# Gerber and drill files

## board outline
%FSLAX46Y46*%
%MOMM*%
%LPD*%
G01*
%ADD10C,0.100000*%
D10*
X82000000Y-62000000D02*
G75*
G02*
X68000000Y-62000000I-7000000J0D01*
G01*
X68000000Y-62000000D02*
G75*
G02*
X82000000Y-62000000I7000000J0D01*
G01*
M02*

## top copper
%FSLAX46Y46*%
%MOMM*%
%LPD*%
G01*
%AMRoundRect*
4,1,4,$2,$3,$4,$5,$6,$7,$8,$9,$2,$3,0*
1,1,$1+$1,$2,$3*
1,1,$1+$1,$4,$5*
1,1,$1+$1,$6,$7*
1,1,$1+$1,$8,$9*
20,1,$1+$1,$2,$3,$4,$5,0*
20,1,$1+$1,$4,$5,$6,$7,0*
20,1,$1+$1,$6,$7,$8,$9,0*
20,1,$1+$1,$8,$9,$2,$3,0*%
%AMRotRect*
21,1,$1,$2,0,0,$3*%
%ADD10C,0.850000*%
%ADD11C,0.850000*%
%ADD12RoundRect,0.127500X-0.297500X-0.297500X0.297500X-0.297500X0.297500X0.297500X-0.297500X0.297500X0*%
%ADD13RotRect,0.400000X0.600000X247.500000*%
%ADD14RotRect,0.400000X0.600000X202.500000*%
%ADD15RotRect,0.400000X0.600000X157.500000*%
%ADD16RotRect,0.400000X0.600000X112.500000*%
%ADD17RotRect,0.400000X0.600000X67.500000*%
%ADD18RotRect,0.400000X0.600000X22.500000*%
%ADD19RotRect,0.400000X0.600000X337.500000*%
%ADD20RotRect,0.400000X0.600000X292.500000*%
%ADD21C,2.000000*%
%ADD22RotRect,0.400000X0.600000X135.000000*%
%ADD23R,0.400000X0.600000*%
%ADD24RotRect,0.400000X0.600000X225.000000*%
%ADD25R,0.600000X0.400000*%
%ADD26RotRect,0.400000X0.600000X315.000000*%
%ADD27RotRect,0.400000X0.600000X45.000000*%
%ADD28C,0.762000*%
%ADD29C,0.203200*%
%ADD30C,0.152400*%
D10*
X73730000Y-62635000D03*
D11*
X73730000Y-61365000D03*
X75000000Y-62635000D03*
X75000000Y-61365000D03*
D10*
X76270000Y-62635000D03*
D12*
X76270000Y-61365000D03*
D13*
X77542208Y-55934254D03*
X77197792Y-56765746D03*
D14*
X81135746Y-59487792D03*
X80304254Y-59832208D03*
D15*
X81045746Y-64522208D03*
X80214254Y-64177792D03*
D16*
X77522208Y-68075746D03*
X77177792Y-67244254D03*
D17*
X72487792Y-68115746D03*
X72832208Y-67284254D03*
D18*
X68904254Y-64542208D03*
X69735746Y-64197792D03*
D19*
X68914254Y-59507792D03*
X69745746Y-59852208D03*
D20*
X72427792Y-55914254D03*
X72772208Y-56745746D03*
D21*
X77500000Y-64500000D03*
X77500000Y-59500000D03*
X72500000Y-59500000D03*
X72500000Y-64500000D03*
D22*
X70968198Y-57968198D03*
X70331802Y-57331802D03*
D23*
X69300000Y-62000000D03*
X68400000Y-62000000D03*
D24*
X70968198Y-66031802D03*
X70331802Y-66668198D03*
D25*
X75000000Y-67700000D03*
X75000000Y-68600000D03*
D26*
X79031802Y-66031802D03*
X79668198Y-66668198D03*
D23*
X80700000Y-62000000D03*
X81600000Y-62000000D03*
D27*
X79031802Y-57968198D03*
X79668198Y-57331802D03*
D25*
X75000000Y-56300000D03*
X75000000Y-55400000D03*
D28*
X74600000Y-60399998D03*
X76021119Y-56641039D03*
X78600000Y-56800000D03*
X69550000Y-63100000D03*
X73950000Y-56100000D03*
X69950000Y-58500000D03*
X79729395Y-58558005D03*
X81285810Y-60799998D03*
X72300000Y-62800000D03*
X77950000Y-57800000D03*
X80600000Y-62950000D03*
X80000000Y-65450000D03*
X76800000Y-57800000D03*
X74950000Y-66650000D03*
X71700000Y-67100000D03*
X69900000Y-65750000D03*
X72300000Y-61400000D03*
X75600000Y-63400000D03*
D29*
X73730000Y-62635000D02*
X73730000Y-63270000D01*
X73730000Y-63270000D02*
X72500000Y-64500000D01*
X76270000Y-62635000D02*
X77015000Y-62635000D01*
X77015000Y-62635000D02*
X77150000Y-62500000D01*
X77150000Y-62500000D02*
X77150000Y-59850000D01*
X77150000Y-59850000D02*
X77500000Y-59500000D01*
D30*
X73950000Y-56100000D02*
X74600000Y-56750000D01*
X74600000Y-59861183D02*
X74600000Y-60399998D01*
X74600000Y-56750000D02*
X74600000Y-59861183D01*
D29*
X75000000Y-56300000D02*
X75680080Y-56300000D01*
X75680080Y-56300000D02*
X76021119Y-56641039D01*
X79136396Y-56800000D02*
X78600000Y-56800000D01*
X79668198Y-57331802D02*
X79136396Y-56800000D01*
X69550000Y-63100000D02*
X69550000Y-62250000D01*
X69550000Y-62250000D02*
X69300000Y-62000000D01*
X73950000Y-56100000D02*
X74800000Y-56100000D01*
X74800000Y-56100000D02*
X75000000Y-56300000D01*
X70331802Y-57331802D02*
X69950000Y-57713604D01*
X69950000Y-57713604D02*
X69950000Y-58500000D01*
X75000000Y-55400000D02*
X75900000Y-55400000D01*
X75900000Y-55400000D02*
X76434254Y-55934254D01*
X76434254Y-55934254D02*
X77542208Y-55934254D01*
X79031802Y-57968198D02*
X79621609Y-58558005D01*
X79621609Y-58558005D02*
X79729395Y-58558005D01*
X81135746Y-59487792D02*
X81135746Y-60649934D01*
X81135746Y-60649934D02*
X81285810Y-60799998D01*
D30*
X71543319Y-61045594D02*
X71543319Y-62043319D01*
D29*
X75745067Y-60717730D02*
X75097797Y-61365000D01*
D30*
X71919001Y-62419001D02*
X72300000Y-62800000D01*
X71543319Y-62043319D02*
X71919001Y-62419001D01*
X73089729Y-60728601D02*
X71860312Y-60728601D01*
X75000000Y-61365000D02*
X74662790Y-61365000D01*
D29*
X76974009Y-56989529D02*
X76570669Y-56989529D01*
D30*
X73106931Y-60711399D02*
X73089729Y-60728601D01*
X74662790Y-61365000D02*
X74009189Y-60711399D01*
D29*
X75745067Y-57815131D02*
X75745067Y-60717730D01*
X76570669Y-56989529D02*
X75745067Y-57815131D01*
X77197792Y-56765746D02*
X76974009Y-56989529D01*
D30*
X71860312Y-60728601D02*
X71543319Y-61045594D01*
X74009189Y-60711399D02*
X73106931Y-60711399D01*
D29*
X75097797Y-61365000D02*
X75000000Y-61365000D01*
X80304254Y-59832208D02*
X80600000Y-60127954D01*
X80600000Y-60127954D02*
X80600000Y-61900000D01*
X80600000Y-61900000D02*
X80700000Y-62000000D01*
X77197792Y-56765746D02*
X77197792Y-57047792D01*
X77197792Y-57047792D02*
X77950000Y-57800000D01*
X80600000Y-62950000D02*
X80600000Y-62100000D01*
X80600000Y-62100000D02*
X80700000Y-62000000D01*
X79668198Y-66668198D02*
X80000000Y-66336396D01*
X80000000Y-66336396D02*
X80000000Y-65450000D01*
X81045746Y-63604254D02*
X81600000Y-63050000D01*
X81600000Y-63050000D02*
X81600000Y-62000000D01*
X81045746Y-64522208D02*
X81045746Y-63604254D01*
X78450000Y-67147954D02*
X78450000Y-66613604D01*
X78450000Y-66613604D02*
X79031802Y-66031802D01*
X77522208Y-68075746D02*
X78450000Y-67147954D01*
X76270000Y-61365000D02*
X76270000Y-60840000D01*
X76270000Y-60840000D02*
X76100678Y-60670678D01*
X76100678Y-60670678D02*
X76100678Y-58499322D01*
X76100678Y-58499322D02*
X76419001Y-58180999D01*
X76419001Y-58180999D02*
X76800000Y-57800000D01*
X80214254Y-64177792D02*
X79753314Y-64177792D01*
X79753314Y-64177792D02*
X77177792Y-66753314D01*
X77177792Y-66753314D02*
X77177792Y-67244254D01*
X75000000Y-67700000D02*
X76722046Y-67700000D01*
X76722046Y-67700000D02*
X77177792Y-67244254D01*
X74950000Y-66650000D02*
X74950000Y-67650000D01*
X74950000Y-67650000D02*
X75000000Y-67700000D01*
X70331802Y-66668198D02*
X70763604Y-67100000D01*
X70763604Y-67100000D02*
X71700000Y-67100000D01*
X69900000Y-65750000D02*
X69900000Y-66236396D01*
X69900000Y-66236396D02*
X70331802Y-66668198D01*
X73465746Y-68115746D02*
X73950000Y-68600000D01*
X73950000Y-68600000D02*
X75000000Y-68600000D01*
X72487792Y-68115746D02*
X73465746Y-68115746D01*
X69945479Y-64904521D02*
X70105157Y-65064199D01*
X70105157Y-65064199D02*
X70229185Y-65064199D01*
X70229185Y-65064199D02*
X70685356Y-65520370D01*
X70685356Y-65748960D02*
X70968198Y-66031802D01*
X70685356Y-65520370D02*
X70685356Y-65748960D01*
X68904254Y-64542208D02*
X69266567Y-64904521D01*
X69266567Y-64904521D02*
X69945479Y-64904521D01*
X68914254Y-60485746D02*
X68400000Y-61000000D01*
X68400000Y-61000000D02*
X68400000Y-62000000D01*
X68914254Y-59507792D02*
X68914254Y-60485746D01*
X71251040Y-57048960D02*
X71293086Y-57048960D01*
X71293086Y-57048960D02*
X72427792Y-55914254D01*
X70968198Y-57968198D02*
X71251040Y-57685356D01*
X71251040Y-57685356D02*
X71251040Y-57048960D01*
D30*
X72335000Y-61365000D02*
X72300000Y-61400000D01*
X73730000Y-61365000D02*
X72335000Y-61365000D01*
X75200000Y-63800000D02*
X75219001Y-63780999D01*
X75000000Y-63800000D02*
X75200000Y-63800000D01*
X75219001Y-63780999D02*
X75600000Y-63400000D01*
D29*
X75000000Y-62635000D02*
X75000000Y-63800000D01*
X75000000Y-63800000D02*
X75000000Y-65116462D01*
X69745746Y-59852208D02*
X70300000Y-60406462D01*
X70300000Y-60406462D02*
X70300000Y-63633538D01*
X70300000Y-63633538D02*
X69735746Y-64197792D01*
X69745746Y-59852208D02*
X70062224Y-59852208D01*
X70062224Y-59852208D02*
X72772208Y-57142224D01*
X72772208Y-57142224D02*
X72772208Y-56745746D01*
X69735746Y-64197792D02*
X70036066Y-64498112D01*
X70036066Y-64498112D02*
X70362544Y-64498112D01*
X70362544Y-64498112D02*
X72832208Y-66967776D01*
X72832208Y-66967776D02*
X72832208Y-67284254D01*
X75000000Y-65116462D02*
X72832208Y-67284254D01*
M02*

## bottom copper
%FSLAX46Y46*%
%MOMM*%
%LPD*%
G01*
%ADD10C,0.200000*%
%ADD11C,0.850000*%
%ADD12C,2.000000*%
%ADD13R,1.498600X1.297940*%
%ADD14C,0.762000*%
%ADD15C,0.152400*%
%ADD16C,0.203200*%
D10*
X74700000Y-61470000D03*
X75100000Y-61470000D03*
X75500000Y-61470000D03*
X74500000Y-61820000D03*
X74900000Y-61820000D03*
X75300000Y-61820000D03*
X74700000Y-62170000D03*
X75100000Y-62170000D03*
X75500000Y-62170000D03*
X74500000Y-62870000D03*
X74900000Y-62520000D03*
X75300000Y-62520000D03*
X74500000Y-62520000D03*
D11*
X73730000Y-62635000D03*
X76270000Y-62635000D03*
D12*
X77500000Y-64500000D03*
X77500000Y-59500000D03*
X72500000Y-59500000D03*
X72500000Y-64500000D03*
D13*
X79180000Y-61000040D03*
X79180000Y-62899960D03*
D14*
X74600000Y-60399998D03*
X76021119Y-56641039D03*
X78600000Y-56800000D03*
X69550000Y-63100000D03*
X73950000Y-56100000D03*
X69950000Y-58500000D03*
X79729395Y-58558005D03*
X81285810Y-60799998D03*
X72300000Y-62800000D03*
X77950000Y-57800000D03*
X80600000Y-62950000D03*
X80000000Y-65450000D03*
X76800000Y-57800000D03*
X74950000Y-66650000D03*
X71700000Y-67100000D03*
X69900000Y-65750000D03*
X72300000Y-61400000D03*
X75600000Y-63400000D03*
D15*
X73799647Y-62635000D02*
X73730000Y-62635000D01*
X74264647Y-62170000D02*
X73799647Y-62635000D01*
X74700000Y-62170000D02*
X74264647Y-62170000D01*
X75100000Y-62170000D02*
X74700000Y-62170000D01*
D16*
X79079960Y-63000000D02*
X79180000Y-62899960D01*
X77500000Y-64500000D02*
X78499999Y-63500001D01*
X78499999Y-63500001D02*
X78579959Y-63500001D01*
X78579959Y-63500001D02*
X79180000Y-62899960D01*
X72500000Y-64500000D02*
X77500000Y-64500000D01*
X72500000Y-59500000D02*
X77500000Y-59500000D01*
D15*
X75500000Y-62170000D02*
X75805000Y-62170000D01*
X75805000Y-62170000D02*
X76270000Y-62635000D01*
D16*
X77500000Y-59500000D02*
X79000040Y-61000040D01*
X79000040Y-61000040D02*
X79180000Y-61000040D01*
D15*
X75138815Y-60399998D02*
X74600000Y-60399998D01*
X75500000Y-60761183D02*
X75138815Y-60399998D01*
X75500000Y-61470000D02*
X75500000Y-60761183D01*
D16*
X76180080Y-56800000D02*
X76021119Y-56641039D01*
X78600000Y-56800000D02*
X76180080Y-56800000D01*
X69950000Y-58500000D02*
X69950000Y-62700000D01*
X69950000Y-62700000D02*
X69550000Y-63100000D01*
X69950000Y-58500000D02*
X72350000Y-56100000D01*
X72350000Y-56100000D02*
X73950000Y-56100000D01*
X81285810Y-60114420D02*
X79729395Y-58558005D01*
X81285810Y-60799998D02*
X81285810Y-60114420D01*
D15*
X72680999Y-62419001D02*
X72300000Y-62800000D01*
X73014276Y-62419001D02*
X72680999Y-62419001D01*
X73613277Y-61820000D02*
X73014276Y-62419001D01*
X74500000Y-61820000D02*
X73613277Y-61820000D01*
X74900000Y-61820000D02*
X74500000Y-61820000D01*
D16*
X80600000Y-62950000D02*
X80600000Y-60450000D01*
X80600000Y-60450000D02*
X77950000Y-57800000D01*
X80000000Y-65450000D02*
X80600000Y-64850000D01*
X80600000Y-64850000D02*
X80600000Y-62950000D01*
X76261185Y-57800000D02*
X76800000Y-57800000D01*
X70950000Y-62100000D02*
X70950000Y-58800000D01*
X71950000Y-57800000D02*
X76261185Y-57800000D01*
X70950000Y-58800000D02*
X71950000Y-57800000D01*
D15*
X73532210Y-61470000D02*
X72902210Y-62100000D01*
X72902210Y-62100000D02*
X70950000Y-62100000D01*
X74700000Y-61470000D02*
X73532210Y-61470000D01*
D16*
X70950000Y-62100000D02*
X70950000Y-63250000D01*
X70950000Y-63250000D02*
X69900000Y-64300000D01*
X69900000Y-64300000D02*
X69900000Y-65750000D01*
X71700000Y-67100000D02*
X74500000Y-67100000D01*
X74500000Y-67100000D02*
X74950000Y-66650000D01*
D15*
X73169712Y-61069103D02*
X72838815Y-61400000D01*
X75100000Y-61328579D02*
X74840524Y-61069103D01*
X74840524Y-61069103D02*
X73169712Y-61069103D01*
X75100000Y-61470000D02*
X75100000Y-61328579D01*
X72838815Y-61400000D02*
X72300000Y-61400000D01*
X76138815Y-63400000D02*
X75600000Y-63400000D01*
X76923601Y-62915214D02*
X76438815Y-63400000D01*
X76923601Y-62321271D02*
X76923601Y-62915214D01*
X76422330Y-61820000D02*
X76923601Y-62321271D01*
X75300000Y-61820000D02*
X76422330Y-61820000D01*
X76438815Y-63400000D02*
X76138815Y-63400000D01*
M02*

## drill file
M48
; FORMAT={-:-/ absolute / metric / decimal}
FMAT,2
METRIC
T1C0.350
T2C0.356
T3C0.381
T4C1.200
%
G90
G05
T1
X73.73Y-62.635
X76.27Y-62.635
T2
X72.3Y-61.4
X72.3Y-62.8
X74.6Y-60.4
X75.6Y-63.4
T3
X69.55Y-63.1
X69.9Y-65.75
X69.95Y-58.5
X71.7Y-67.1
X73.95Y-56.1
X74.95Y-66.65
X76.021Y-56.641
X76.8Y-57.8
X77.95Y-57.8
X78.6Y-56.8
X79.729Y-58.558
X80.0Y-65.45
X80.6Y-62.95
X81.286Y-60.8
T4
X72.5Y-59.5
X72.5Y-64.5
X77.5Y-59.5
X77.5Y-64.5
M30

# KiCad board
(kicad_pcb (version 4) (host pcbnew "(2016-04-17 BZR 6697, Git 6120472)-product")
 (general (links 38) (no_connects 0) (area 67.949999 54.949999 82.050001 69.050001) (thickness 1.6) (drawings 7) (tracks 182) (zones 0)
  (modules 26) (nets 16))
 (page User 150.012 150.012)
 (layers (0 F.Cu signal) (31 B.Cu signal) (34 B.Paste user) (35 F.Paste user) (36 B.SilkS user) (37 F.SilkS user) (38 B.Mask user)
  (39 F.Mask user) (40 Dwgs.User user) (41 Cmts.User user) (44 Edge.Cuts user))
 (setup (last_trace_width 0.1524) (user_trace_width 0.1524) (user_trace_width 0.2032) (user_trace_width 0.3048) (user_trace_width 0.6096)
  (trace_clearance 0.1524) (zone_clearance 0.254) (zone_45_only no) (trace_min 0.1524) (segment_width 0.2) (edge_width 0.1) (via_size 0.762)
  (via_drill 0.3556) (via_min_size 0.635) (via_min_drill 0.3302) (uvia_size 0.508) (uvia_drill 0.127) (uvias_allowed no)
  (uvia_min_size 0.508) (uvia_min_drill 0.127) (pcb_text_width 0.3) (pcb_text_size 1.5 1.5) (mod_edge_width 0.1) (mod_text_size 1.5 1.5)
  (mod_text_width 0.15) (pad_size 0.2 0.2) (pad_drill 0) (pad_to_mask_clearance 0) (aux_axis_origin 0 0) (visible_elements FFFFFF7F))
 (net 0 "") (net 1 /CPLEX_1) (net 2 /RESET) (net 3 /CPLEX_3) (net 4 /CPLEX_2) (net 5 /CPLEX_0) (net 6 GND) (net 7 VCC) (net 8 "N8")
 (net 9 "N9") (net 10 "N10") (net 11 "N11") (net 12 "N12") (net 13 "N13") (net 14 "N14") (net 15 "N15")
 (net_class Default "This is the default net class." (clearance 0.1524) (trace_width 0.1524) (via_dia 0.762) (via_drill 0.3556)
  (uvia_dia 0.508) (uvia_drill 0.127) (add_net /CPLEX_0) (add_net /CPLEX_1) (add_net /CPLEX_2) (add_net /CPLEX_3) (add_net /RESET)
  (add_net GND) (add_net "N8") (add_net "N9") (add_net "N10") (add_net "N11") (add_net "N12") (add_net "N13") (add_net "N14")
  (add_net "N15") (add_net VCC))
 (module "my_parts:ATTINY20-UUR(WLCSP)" (layer B.Cu) (at 75 62) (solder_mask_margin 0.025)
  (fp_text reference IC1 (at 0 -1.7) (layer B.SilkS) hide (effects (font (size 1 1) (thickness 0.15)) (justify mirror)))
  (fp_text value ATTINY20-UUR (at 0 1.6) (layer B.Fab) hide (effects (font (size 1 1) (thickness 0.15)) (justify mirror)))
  (pad D2 smd circle (at -0.3 -0.53) (size 0.2 0.2) (layers B.Cu B.Paste B.Mask) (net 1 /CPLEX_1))
  (pad D4 smd circle (at 0.1 -0.53) (size 0.2 0.2) (layers B.Cu B.Paste B.Mask) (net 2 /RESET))
  (pad D6 smd circle (at 0.5 -0.53) (size 0.2 0.2) (layers B.Cu B.Paste B.Mask) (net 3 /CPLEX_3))
  (pad C1 smd circle (at -0.5 -0.18) (size 0.2 0.2) (layers B.Cu B.Paste B.Mask) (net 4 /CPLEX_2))
  (pad C3 smd circle (at -0.1 -0.18) (size 0.2 0.2) (layers B.Cu B.Paste B.Mask) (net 4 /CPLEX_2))
  (pad C5 smd circle (at 0.3 -0.18) (size 0.2 0.2) (layers B.Cu B.Paste B.Mask) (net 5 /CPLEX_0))
  (pad B2 smd circle (at -0.3 0.17) (size 0.2 0.2) (layers B.Cu B.Paste B.Mask) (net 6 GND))
  (pad B4 smd circle (at 0.1 0.17) (size 0.2 0.2) (layers B.Cu B.Paste B.Mask) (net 6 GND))
  (pad B6 smd circle (at 0.5 0.17) (size 0.2 0.2) (layers B.Cu B.Paste B.Mask) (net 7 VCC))
  (pad A1 smd circle (at -0.5 0.87) (size 0.2 0.2) (layers B.Cu))
  (pad A3 smd circle (at -0.1 0.52) (size 0.2 0.2) (layers B.Cu B.Paste B.Mask))
  (pad A5 smd circle (at 0.3 0.52) (size 0.2 0.2) (layers B.Cu B.Paste B.Mask))
  (pad A1 smd circle (at -0.5 0.52) (size 0.2 0.2) (layers B.Cu B.Paste B.Mask)))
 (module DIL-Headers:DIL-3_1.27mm (layer F.Cu) (at 75 62) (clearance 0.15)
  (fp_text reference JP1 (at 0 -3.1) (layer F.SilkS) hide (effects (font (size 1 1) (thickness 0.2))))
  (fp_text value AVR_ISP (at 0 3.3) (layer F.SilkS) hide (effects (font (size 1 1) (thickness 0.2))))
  (pad 6 thru_hole circle (at -1.27 0.635) (size 0.85 0.85) (drill 0.35) (layers *.Cu F.Mask) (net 6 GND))
  (pad 5 smd circle (at -1.27 -0.635) (size 0.85 0.85) (layers F.Cu F.Mask) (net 2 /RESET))
  (pad 4 smd circle (at 0 0.635) (size 0.85 0.85) (layers F.Cu F.Mask) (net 5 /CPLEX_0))
  (pad 3 smd circle (at 0 -0.635) (size 0.85 0.85) (layers F.Cu F.Mask) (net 4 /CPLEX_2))
  (pad 2 thru_hole circle (at 1.27 0.635) (size 0.85 0.85) (drill 0.35) (layers *.Cu F.Mask) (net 7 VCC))
  (pad 1 smd roundrect (at 1.27 -0.635) (size 0.85 0.85) (layers F.Cu F.Mask) (roundrect_rratio 0.15) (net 1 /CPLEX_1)))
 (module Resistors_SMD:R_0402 (layer F.Cu) (at 77.37 56.35 247.5)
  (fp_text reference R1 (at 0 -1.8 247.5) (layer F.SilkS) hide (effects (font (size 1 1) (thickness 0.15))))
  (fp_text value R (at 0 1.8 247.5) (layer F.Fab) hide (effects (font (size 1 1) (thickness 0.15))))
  (pad 1 smd rect (at -0.45 0 247.5) (size 0.4 0.6) (layers F.Cu F.Paste F.Mask) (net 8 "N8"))
  (pad 2 smd rect (at 0.45 0 247.5) (size 0.4 0.6) (layers F.Cu F.Paste F.Mask) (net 4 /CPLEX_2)))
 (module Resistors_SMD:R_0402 (layer F.Cu) (at 80.72 59.66 202.5)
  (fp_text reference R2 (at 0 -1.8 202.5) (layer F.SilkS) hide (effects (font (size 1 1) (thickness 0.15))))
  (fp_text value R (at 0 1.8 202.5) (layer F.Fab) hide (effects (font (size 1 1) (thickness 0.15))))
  (pad 1 smd rect (at -0.45 0 202.5) (size 0.4 0.6) (layers F.Cu F.Paste F.Mask) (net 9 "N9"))
  (pad 2 smd rect (at 0.45 0 202.5) (size 0.4 0.6) (layers F.Cu F.Paste F.Mask) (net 4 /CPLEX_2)))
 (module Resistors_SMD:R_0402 (layer F.Cu) (at 80.63 64.35 157.5)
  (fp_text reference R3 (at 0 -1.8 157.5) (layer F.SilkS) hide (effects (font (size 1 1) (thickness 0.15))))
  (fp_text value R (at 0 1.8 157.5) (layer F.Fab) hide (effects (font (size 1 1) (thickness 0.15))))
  (pad 1 smd rect (at -0.45 0 157.5) (size 0.4 0.6) (layers F.Cu F.Paste F.Mask) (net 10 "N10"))
  (pad 2 smd rect (at 0.45 0 157.5) (size 0.4 0.6) (layers F.Cu F.Paste F.Mask) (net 1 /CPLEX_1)))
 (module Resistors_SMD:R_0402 (layer F.Cu) (at 77.35 67.66 112.5)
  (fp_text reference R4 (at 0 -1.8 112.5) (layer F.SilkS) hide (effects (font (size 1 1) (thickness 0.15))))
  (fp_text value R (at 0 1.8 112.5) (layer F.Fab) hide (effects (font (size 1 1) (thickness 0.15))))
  (pad 1 smd rect (at -0.45 0 112.5) (size 0.4 0.6) (layers F.Cu F.Paste F.Mask) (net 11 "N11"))
  (pad 2 smd rect (at 0.45 0 112.5) (size 0.4 0.6) (layers F.Cu F.Paste F.Mask) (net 1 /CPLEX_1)))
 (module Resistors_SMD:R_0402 (layer F.Cu) (at 72.66 67.7 67.5)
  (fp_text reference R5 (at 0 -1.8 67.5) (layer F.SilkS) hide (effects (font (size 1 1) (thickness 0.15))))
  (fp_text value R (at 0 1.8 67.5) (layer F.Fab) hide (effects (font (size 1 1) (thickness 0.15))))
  (pad 1 smd rect (at -0.45 0 67.5) (size 0.4 0.6) (layers F.Cu F.Paste F.Mask) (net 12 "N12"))
  (pad 2 smd rect (at 0.45 0 67.5) (size 0.4 0.6) (layers F.Cu F.Paste F.Mask) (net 5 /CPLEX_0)))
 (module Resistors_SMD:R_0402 (layer F.Cu) (at 69.32 64.37 22.5)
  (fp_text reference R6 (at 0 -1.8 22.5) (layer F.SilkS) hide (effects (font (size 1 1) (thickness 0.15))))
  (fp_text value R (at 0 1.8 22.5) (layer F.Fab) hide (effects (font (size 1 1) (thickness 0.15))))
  (pad 1 smd rect (at -0.45 0 22.5) (size 0.4 0.6) (layers F.Cu F.Paste F.Mask) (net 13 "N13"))
  (pad 2 smd rect (at 0.45 0 22.5) (size 0.4 0.6) (layers F.Cu F.Paste F.Mask) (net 5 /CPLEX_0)))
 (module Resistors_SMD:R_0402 (layer F.Cu) (at 69.33 59.68 337.5)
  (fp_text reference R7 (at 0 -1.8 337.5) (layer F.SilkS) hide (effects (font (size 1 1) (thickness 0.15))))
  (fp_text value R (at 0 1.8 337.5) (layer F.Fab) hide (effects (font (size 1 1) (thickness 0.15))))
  (pad 1 smd rect (at -0.45 0 337.5) (size 0.4 0.6) (layers F.Cu F.Paste F.Mask) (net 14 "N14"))
  (pad 2 smd rect (at 0.45 0 337.5) (size 0.4 0.6) (layers F.Cu F.Paste F.Mask) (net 5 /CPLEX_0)))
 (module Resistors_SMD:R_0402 (layer F.Cu) (at 72.6 56.33 292.5)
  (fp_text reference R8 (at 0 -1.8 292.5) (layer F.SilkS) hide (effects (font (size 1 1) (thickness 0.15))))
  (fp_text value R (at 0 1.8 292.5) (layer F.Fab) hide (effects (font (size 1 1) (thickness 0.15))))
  (pad 1 smd rect (at -0.45 0 292.5) (size 0.4 0.6) (layers F.Cu F.Paste F.Mask) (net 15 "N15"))
  (pad 2 smd rect (at 0.45 0 292.5) (size 0.4 0.6) (layers F.Cu F.Paste F.Mask) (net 5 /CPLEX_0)))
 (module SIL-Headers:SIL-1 (layer F.Cu) (at 77.5 64.5)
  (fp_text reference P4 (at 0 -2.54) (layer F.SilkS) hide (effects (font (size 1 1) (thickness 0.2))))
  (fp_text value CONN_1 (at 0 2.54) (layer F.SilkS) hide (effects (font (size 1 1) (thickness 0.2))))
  (pad 1 thru_hole circle (at 0 0) (size 2 2) (drill 1.2) (layers *.Cu *.Mask) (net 6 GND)))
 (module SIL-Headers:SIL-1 (layer F.Cu) (at 77.5 59.5)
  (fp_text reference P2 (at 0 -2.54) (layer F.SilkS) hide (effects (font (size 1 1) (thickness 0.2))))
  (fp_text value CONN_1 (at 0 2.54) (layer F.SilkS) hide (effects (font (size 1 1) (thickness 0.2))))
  (pad 1 thru_hole circle (at 0 0) (size 2 2) (drill 1.2) (layers *.Cu *.Mask) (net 7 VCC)))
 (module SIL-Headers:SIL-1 (layer F.Cu) (at 72.5 59.5)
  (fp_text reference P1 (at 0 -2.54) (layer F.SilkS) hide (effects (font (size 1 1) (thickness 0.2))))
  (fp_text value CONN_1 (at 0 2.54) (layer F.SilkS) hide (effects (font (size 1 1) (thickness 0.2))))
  (pad 1 thru_hole circle (at 0 0) (size 2 2) (drill 1.2) (layers *.Cu *.Mask) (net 7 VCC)))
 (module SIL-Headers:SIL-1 (layer F.Cu) (at 72.5 64.5)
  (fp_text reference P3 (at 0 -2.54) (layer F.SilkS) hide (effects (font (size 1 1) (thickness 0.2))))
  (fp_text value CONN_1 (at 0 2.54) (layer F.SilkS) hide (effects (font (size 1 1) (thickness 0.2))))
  (pad 1 thru_hole circle (at 0 0) (size 2 2) (drill 1.2) (layers *.Cu *.Mask) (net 6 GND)))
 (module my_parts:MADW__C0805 (layer B.Cu) (at 79.18 61.95 270)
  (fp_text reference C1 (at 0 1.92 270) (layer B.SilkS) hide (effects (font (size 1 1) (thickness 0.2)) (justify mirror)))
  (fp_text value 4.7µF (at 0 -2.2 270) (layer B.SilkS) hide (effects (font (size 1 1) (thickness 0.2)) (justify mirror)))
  (pad 1 smd rect (at -0.94996 0 270) (size 1.29794 1.4986) (layers B.Cu B.Paste B.Mask) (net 7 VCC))
  (pad 2 smd rect (at 0.94996 0 270) (size 1.29794 1.4986) (layers B.Cu B.Paste B.Mask) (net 6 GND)))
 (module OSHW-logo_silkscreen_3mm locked (layer B.Cu) (at 75 56.8)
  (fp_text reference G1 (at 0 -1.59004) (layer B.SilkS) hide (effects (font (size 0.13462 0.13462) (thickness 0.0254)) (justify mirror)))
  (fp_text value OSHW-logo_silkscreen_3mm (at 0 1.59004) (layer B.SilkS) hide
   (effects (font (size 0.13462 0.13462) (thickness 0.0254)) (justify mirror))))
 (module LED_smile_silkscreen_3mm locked (layer B.Cu) (at 75 67.2)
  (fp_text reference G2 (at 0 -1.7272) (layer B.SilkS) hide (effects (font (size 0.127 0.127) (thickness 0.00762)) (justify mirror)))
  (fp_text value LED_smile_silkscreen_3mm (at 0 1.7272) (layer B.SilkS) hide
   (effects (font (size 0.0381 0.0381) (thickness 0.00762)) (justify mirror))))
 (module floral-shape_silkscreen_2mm (layer F.Cu) (at 75.03 57.9 45)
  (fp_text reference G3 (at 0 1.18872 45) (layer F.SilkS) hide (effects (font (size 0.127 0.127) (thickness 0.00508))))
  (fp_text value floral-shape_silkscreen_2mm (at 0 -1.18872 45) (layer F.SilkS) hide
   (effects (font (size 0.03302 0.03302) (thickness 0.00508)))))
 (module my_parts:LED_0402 (layer F.Cu) (at 70.65 57.65 135)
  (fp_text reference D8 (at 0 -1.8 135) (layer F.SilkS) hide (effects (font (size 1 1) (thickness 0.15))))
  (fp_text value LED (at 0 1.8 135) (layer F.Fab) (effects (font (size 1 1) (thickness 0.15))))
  (pad 1 smd rect (at -0.45 0 135) (size 0.4 0.6) (layers F.Cu F.Paste F.Mask) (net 15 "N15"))
  (pad 2 smd rect (at 0.45 0 135) (size 0.4 0.6) (layers F.Cu F.Paste F.Mask) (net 3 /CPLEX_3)))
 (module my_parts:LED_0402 (layer F.Cu) (at 68.85 62 180)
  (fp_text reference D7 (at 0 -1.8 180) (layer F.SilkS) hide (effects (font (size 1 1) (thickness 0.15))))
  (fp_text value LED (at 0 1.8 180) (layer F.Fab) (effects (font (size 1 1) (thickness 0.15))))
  (pad 1 smd rect (at -0.45 0 180) (size 0.4 0.6) (layers F.Cu F.Paste F.Mask) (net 3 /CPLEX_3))
  (pad 2 smd rect (at 0.45 0 180) (size 0.4 0.6) (layers F.Cu F.Paste F.Mask) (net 14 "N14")))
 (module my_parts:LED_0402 (layer F.Cu) (at 70.65 66.35 225)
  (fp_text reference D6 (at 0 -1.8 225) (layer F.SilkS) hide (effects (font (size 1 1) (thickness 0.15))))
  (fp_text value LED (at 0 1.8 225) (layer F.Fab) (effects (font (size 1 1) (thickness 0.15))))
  (pad 1 smd rect (at -0.45 0 225) (size 0.4 0.6) (layers F.Cu F.Paste F.Mask) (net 13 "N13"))
  (pad 2 smd rect (at 0.45 0 225) (size 0.4 0.6) (layers F.Cu F.Paste F.Mask) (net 1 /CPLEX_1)))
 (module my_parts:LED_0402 (layer F.Cu) (at 75 68.15 270)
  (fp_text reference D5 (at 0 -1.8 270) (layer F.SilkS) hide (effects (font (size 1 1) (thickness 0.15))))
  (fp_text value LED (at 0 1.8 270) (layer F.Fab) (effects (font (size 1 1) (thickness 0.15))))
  (pad 1 smd rect (at -0.45 0 270) (size 0.4 0.6) (layers F.Cu F.Paste F.Mask) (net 1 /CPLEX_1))
  (pad 2 smd rect (at 0.45 0 270) (size 0.4 0.6) (layers F.Cu F.Paste F.Mask) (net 12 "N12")))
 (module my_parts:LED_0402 (layer F.Cu) (at 79.35 66.35 315)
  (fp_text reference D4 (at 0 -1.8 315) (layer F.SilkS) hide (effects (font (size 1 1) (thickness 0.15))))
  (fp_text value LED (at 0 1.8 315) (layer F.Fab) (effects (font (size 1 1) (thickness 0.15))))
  (pad 1 smd rect (at -0.45 0 315) (size 0.4 0.6) (layers F.Cu F.Paste F.Mask) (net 11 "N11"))
  (pad 2 smd rect (at 0.45 0 315) (size 0.4 0.6) (layers F.Cu F.Paste F.Mask) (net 4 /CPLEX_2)))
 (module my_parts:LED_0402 (layer F.Cu) (at 81.15 62)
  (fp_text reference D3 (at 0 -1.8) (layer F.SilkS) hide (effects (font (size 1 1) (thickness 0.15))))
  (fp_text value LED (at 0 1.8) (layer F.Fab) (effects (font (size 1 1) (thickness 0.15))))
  (pad 1 smd rect (at -0.45 0) (size 0.4 0.6) (layers F.Cu F.Paste F.Mask) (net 4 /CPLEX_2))
  (pad 2 smd rect (at 0.45 0) (size 0.4 0.6) (layers F.Cu F.Paste F.Mask) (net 10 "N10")))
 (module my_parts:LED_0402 (layer F.Cu) (at 79.35 57.65 45)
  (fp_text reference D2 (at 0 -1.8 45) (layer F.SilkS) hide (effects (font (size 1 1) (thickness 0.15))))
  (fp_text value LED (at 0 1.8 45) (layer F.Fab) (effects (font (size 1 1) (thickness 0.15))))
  (pad 1 smd rect (at -0.45 0 45) (size 0.4 0.6) (layers F.Cu F.Paste F.Mask) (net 9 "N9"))
  (pad 2 smd rect (at 0.45 0 45) (size 0.4 0.6) (layers F.Cu F.Paste F.Mask) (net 3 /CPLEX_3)))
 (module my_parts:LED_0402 (layer F.Cu) (at 75 55.85 90)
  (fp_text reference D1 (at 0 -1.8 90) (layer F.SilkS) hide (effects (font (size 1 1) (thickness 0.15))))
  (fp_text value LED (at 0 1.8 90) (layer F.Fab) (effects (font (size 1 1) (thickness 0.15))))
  (pad 1 smd rect (at -0.45 0 90) (size 0.4 0.6) (layers F.Cu F.Paste F.Mask) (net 3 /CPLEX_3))
  (pad 2 smd rect (at 0.45 0 90) (size 0.4 0.6) (layers F.Cu F.Paste F.Mask) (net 8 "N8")))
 (gr_circle (center 75 62) (end 82 62) (layer Edge.Cuts) (width 0.1))
 (segment (start 73.799647 62.635) (end 73.73 62.635) (width 0.1524) (layer B.Cu) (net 6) (status 30))
 (segment (start 74.264647 62.17) (end 73.799647 62.635) (width 0.1524) (layer B.Cu) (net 6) (status 20))
 (segment (start 74.7 62.17) (end 74.264647 62.17) (width 0.1524) (layer B.Cu) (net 6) (status 10))
 (segment (start 75.1 62.17) (end 74.7 62.17) (width 0.1524) (layer B.Cu) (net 6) (status 30))
 (segment (start 73.73 62.635) (end 73.73 63.27) (width 0.2032) (layer F.Cu) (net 6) (status 10))
 (segment (start 73.73 63.27) (end 72.5 64.5) (width 0.2032) (layer F.Cu) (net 6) (status 20))
 (segment (start 79.07996 63) (end 79.18 62.89996) (width 0.2032) (layer B.Cu) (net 6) (status 30))
 (segment (start 77.5 64.5) (end 78.499999 63.500001) (width 0.2032) (layer B.Cu) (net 6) (status 30))
 (segment (start 78.499999 63.500001) (end 78.579959 63.500001) (width 0.2032) (layer B.Cu) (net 6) (status 30))
 (segment (start 78.579959 63.500001) (end 79.18 62.89996) (width 0.2032) (layer B.Cu) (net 6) (status 30))
 (segment (start 72.5 64.5) (end 77.5 64.5) (width 0.2032) (layer B.Cu) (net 6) (status 30))
 (segment (start 72.5 59.5) (end 77.5 59.5) (width 0.2032) (layer B.Cu) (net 7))
 (segment (start 75.5 62.17) (end 75.805 62.17) (width 0.1524) (layer B.Cu) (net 7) (status 10))
 (segment (start 75.805 62.17) (end 76.27 62.635) (width 0.1524) (layer B.Cu) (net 7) (status 20))
 (segment (start 76.27 62.635) (end 77.015 62.635) (width 0.2032) (layer F.Cu) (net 7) (status 10))
 (segment (start 77.015 62.635) (end 77.15 62.5) (width 0.2032) (layer F.Cu) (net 7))
 (segment (start 77.15 62.5) (end 77.15 59.85) (width 0.2032) (layer F.Cu) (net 7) (status 20))
 (segment (start 77.15 59.85) (end 77.5 59.5) (width 0.2032) (layer F.Cu) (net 7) (status 30))
 (segment (start 77.5 59.5) (end 79.00004 61.00004) (width 0.2032) (layer B.Cu) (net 7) (status 30))
 (segment (start 79.00004 61.00004) (end 79.18 61.00004) (width 0.2032) (layer B.Cu) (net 7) (status 30))
 (segment (start 73.95 56.1) (end 74.6 56.75) (width 0.1524) (layer F.Cu) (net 3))
 (segment (start 75.138815 60.399998) (end 74.6 60.399998) (width 0.1524) (layer B.Cu) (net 3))
 (segment (start 75.5 60.761183) (end 75.138815 60.399998) (width 0.1524) (layer B.Cu) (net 3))
 (segment (start 74.6 59.861183) (end 74.6 60.399998) (width 0.1524) (layer F.Cu) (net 3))
 (segment (start 74.6 56.75) (end 74.6 59.861183) (width 0.1524) (layer F.Cu) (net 3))
 (segment (start 75.5 61.47) (end 75.5 60.761183) (width 0.1524) (layer B.Cu) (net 3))
 (via (at 74.6 60.399998) (size 0.762) (drill 0.3556) (layers F.Cu B.Cu) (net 3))
 (segment (start 75 56.3) (end 75.68008 56.3) (width 0.2032) (layer F.Cu) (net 3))
 (segment (start 76.18008 56.8) (end 76.021119 56.641039) (width 0.2032) (layer B.Cu) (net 3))
 (segment (start 75.68008 56.3) (end 76.021119 56.641039) (width 0.2032) (layer F.Cu) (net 3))
 (segment (start 78.6 56.8) (end 76.18008 56.8) (width 0.2032) (layer B.Cu) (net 3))
 (via (at 76.021119 56.641039) (size 0.762) (drill 0.381) (layers F.Cu B.Cu) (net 3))
 (segment (start 79.136396 56.8) (end 78.6 56.8) (width 0.2032) (layer F.Cu) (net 3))
 (segment (start 79.668198 57.331802) (end 79.136396 56.8) (width 0.2032) (layer F.Cu) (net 3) (status 10))
 (via (at 78.6 56.8) (size 0.762) (drill 0.381) (layers F.Cu B.Cu) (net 3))
 (segment (start 69.55 63.1) (end 69.55 62.25) (width 0.2032) (layer F.Cu) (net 3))
 (segment (start 69.55 62.25) (end 69.3 62) (width 0.2032) (layer F.Cu) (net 3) (status 20))
 (segment (start 69.95 58.5) (end 69.95 62.7) (width 0.2032) (layer B.Cu) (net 3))
 (segment (start 69.95 62.7) (end 69.55 63.1) (width 0.2032) (layer B.Cu) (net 3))
 (via (at 69.55 63.1) (size 0.762) (drill 0.381) (layers F.Cu B.Cu) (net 3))
 (segment (start 73.95 56.1) (end 74.8 56.1) (width 0.2032) (layer F.Cu) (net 3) (status 20))
 (segment (start 74.8 56.1) (end 75 56.3) (width 0.2032) (layer F.Cu) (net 3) (status 30))
 (segment (start 69.95 58.5) (end 72.35 56.1) (width 0.2032) (layer B.Cu) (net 3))
 (segment (start 72.35 56.1) (end 73.95 56.1) (width 0.2032) (layer B.Cu) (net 3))
 (via (at 73.95 56.1) (size 0.762) (drill 0.381) (layers F.Cu B.Cu) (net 3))
 (segment (start 70.331802 57.331802) (end 69.95 57.713604) (width 0.2032) (layer F.Cu) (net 3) (status 10))
 (segment (start 69.95 57.713604) (end 69.95 58.5) (width 0.2032) (layer F.Cu) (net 3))
 (via (at 69.95 58.5) (size 0.762) (drill 0.381) (layers F.Cu B.Cu) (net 3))
 (segment (start 75 55.4) (end 75.9 55.4) (width 0.2032) (layer F.Cu) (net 8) (status 10))
 (segment (start 75.9 55.4) (end 76.434254 55.934254) (width 0.2032) (layer F.Cu) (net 8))
 (segment (start 76.434254 55.934254) (end 77.542208 55.934254) (width 0.2032) (layer F.Cu) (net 8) (status 20))
 (segment (start 81.28581 60.11442) (end 79.729395 58.558005) (width 0.2032) (layer B.Cu) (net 9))
 (segment (start 81.28581 60.799998) (end 81.28581 60.11442) (width 0.2032) (layer B.Cu) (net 9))
 (segment (start 79.031802 57.968198) (end 79.621609 58.558005) (width 0.2032) (layer F.Cu) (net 9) (status 10))
 (segment (start 79.621609 58.558005) (end 79.729395 58.558005) (width 0.2032) (layer F.Cu) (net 9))
 (via (at 79.729395 58.558005) (size 0.762) (drill 0.381) (layers F.Cu B.Cu) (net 9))
 (segment (start 81.135746 59.487792) (end 81.135746 60.649934) (width 0.2032) (layer F.Cu) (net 9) (status 10))
 (via (at 81.28581 60.799998) (size 0.762) (drill 0.381) (layers F.Cu B.Cu) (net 9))
 (segment (start 81.135746 60.649934) (end 81.28581 60.799998) (width 0.2032) (layer F.Cu) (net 9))
 (segment (start 71.543319 61.045594) (end 71.543319 62.043319) (width 0.1524) (layer F.Cu) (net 4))
 (segment (start 75.745067 60.71773) (end 75.097797 61.365) (width 0.2032) (layer F.Cu) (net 4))
 (segment (start 71.919001 62.419001) (end 72.3 62.8) (width 0.1524) (layer F.Cu) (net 4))
 (segment (start 71.543319 62.043319) (end 71.919001 62.419001) (width 0.1524) (layer F.Cu) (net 4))
 (segment (start 73.089729 60.728601) (end 71.860312 60.728601) (width 0.1524) (layer F.Cu) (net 4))
 (segment (start 75 61.365) (end 74.66279 61.365) (width 0.1524) (layer F.Cu) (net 4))
 (segment (start 76.974009 56.989529) (end 76.570669 56.989529) (width 0.2032) (layer F.Cu) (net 4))
 (segment (start 73.106931 60.711399) (end 73.089729 60.728601) (width 0.1524) (layer F.Cu) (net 4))
 (segment (start 74.66279 61.365) (end 74.009189 60.711399) (width 0.1524) (layer F.Cu) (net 4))
 (segment (start 75.745067 57.815131) (end 75.745067 60.71773) (width 0.2032) (layer F.Cu) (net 4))
 (segment (start 76.570669 56.989529) (end 75.745067 57.815131) (width 0.2032) (layer F.Cu) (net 4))
 (segment (start 77.197792 56.765746) (end 76.974009 56.989529) (width 0.2032) (layer F.Cu) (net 4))
 (segment (start 71.860312 60.728601) (end 71.543319 61.045594) (width 0.1524) (layer F.Cu) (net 4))
 (segment (start 74.009189 60.711399) (end 73.106931 60.711399) (width 0.1524) (layer F.Cu) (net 4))
 (segment (start 75.097797 61.365) (end 75 61.365) (width 0.2032) (layer F.Cu) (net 4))
 (segment (start 72.680999 62.419001) (end 72.3 62.8) (width 0.1524) (layer B.Cu) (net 4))
 (segment (start 73.014276 62.419001) (end 72.680999 62.419001) (width 0.1524) (layer B.Cu) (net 4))
 (segment (start 73.613277 61.82) (end 73.014276 62.419001) (width 0.1524) (layer B.Cu) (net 4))
 (segment (start 74.5 61.82) (end 73.613277 61.82) (width 0.1524) (layer B.Cu) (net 4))
 (via (at 72.3 62.8) (size 0.762) (drill 0.3556) (layers F.Cu B.Cu) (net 4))
 (segment (start 74.9 61.82) (end 74.5 61.82) (width 0.1524) (layer B.Cu) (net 4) (status 30))
 (segment (start 80.6 62.95) (end 80.6 60.45) (width 0.2032) (layer B.Cu) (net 4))
 (segment (start 80.6 60.45) (end 77.95 57.8) (width 0.2032) (layer B.Cu) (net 4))
 (segment (start 80.304254 59.832208) (end 80.6 60.127954) (width 0.2032) (layer F.Cu) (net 4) (status 10))
 (segment (start 80.6 60.127954) (end 80.6 61.9) (width 0.2032) (layer F.Cu) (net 4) (status 20))
 (segment (start 80.6 61.9) (end 80.7 62) (width 0.2032) (layer F.Cu) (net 4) (status 30))
 (segment (start 77.197792 56.765746) (end 77.197792 57.047792) (width 0.2032) (layer F.Cu) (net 4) (status 10))
 (segment (start 77.197792 57.047792) (end 77.95 57.8) (width 0.2032) (layer F.Cu) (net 4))
 (via (at 77.95 57.8) (size 0.762) (drill 0.381) (layers F.Cu B.Cu) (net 4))
 (segment (start 80.6 62.95) (end 80.6 62.1) (width 0.2032) (layer F.Cu) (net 4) (status 20))
 (segment (start 80.6 62.1) (end 80.7 62) (width 0.2032) (layer F.Cu) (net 4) (status 30))
 (segment (start 80 65.45) (end 80.6 64.85) (width 0.2032) (layer B.Cu) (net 4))
 (via (at 80.6 62.95) (size 0.762) (drill 0.381) (layers F.Cu B.Cu) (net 4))
 (segment (start 80.6 64.85) (end 80.6 62.95) (width 0.2032) (layer B.Cu) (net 4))
 (segment (start 79.668198 66.668198) (end 80 66.336396) (width 0.2032) (layer F.Cu) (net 4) (status 10))
 (segment (start 80 66.336396) (end 80 65.45) (width 0.2032) (layer F.Cu) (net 4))
 (via (at 80 65.45) (size 0.762) (drill 0.381) (layers F.Cu B.Cu) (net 4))
 (segment (start 81.045746 63.604254) (end 81.6 63.05) (width 0.2032) (layer F.Cu) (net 10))
 (segment (start 81.6 63.05) (end 81.6 62) (width 0.2032) (layer F.Cu) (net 10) (status 20))
 (segment (start 81.045746 64.522208) (end 81.045746 63.604254) (width 0.2032) (layer F.Cu) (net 10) (status 10))
 (segment (start 78.45 67.147954) (end 78.45 66.613604) (width 0.2032) (layer F.Cu) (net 11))
 (segment (start 78.45 66.613604) (end 79.031802 66.031802) (width 0.2032) (layer F.Cu) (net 11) (status 20))
 (segment (start 77.522208 68.075746) (end 78.45 67.147954) (width 0.2032) (layer F.Cu) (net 11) (status 10))
 (segment (start 76.27 61.365) (end 76.27 60.84) (width 0.2032) (layer F.Cu) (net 1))
 (segment (start 76.27 60.84) (end 76.100678 60.670678) (width 0.2032) (layer F.Cu) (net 1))
 (segment (start 76.100678 60.670678) (end 76.100678 58.499322) (width 0.2032) (layer F.Cu) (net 1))
 (segment (start 76.100678 58.499322) (end 76.419001 58.180999) (width 0.2032) (layer F.Cu) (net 1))
 (segment (start 76.419001 58.180999) (end 76.8 57.8) (width 0.2032) (layer F.Cu) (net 1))
 (segment (start 76.261185 57.8) (end 76.8 57.8) (width 0.2032) (layer B.Cu) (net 1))
 (segment (start 70.95 62.1) (end 70.95 58.8) (width 0.2032) (layer B.Cu) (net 1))
 (via (at 76.8 57.8) (size 0.762) (drill 0.381) (layers F.Cu B.Cu) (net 1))
 (segment (start 71.95 57.8) (end 76.261185 57.8) (width 0.2032) (layer B.Cu) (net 1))
 (segment (start 70.95 58.8) (end 71.95 57.8) (width 0.2032) (layer B.Cu) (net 1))
 (segment (start 73.53221 61.47) (end 72.90221 62.1) (width 0.1524) (layer B.Cu) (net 1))
 (segment (start 72.90221 62.1) (end 70.95 62.1) (width 0.1524) (layer B.Cu) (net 1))
 (segment (start 74.7 61.47) (end 73.53221 61.47) (width 0.1524) (layer B.Cu) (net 1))
 (segment (start 70.95 62.1) (end 70.95 63.25) (width 0.2032) (layer B.Cu) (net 1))
 (segment (start 70.95 63.25) (end 69.9 64.3) (width 0.2032) (layer B.Cu) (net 1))
 (segment (start 69.9 64.3) (end 69.9 65.75) (width 0.2032) (layer B.Cu) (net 1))
 (segment (start 80.214254 64.177792) (end 79.753314 64.177792) (width 0.2032) (layer F.Cu) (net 1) (status 10))
 (segment (start 79.753314 64.177792) (end 77.177792 66.753314) (width 0.2032) (layer F.Cu) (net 1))
 (segment (start 77.177792 66.753314) (end 77.177792 67.244254) (width 0.2032) (layer F.Cu) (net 1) (status 20))
 (segment (start 75 67.7) (end 76.722046 67.7) (width 0.2032) (layer F.Cu) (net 1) (status 10))
 (segment (start 76.722046 67.7) (end 77.177792 67.244254) (width 0.2032) (layer F.Cu) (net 1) (status 20))
 (segment (start 74.95 66.65) (end 74.95 67.65) (width 0.2032) (layer F.Cu) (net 1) (status 20))
 (segment (start 74.95 67.65) (end 75 67.7) (width 0.2032) (layer F.Cu) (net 1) (status 30))
 (segment (start 71.7 67.1) (end 74.5 67.1) (width 0.2032) (layer B.Cu) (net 1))
 (via (at 74.95 66.65) (size 0.762) (drill 0.381) (layers F.Cu B.Cu) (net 1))
 (segment (start 74.5 67.1) (end 74.95 66.65) (width 0.2032) (layer B.Cu) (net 1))
 (segment (start 70.331802 66.668198) (end 70.763604 67.1) (width 0.2032) (layer F.Cu) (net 1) (status 10))
 (segment (start 70.763604 67.1) (end 71.7 67.1) (width 0.2032) (layer F.Cu) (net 1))
 (via (at 71.7 67.1) (size 0.762) (drill 0.381) (layers F.Cu B.Cu) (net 1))
 (segment (start 69.9 65.75) (end 69.9 66.236396) (width 0.2032) (layer F.Cu) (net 1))
 (segment (start 69.9 66.236396) (end 70.331802 66.668198) (width 0.2032) (layer F.Cu) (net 1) (status 20))
 (via (at 69.9 65.75) (size 0.762) (drill 0.381) (layers F.Cu B.Cu) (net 1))
 (segment (start 73.465746 68.115746) (end 73.95 68.6) (width 0.2032) (layer F.Cu) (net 12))
 (segment (start 73.95 68.6) (end 75 68.6) (width 0.2032) (layer F.Cu) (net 12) (status 20))
 (segment (start 72.487792 68.115746) (end 73.465746 68.115746) (width 0.2032) (layer F.Cu) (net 12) (status 10))
 (segment (start 69.945479 64.904521) (end 70.105157 65.064199) (width 0.2032) (layer F.Cu) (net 13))
 (segment (start 70.105157 65.064199) (end 70.229185 65.064199) (width 0.2032) (layer F.Cu) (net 13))
 (segment (start 70.229185 65.064199) (end 70.685356 65.52037) (width 0.2032) (layer F.Cu) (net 13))
 (segment (start 70.685356 65.74896) (end 70.968198 66.031802) (width 0.2032) (layer F.Cu) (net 13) (status 20))
 (segment (start 70.685356 65.52037) (end 70.685356 65.74896) (width 0.2032) (layer F.Cu) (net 13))
 (segment (start 68.904254 64.542208) (end 69.266567 64.904521) (width 0.2032) (layer F.Cu) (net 13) (status 10))
 (segment (start 69.266567 64.904521) (end 69.945479 64.904521) (width 0.2032) (layer F.Cu) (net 13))
 (segment (start 68.914254 60.485746) (end 68.4 61) (width 0.2032) (layer F.Cu) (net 14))
 (segment (start 68.4 61) (end 68.4 62) (width 0.2032) (layer F.Cu) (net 14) (status 20))
 (segment (start 68.914254 59.507792) (end 68.914254 60.485746) (width 0.2032) (layer F.Cu) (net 14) (status 10))
 (segment (start 71.25104 57.04896) (end 71.293086 57.04896) (width 0.2032) (layer F.Cu) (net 15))
 (segment (start 71.293086 57.04896) (end 72.427792 55.914254) (width 0.2032) (layer F.Cu) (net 15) (status 20))
 (segment (start 70.968198 57.968198) (end 71.25104 57.685356) (width 0.2032) (layer F.Cu) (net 15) (status 10))
 (segment (start 71.25104 57.685356) (end 71.25104 57.04896) (width 0.2032) (layer F.Cu) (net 15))
 (segment (start 73.169712 61.069103) (end 72.838815 61.4) (width 0.1524) (layer B.Cu) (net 2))
 (segment (start 75.1 61.328579) (end 74.840524 61.069103) (width 0.1524) (layer B.Cu) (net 2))
 (segment (start 74.840524 61.069103) (end 73.169712 61.069103) (width 0.1524) (layer B.Cu) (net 2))
 (segment (start 75.1 61.47) (end 75.1 61.328579) (width 0.1524) (layer B.Cu) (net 2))
 (segment (start 72.838815 61.4) (end 72.3 61.4) (width 0.1524) (layer B.Cu) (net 2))
 (segment (start 72.335 61.365) (end 72.3 61.4) (width 0.1524) (layer F.Cu) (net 2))
 (via (at 72.3 61.4) (size 0.762) (drill 0.3556) (layers F.Cu B.Cu) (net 2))
 (segment (start 73.73 61.365) (end 72.335 61.365) (width 0.1524) (layer F.Cu) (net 2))
 (segment (start 76.138815 63.4) (end 75.6 63.4) (width 0.1524) (layer B.Cu) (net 5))
 (segment (start 76.923601 62.915214) (end 76.438815 63.4) (width 0.1524) (layer B.Cu) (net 5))
 (segment (start 76.923601 62.321271) (end 76.923601 62.915214) (width 0.1524) (layer B.Cu) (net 5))
 (segment (start 76.42233 61.82) (end 76.923601 62.321271) (width 0.1524) (layer B.Cu) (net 5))
 (segment (start 75.3 61.82) (end 76.42233 61.82) (width 0.1524) (layer B.Cu) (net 5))
 (segment (start 75.2 63.8) (end 75.219001 63.780999) (width 0.1524) (layer F.Cu) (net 5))
 (segment (start 75 63.8) (end 75.2 63.8) (width 0.1524) (layer F.Cu) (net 5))
 (segment (start 75.219001 63.780999) (end 75.6 63.4) (width 0.1524) (layer F.Cu) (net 5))
 (segment (start 76.438815 63.4) (end 76.138815 63.4) (width 0.1524) (layer B.Cu) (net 5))
 (via (at 75.6 63.4) (size 0.762) (drill 0.3556) (layers F.Cu B.Cu) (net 5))
 (segment (start 75 62.635) (end 75 63.8) (width 0.2032) (layer F.Cu) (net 5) (status 10))
 (segment (start 75 63.8) (end 75 65.116462) (width 0.2032) (layer F.Cu) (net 5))
 (segment (start 69.745746 59.852208) (end 70.3 60.406462) (width 0.2032) (layer F.Cu) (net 5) (status 10))
 (segment (start 70.3 60.406462) (end 70.3 63.633538) (width 0.2032) (layer F.Cu) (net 5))
 (segment (start 70.3 63.633538) (end 69.735746 64.197792) (width 0.2032) (layer F.Cu) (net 5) (status 20))
 (segment (start 69.745746 59.852208) (end 70.062224 59.852208) (width 0.2032) (layer F.Cu) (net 5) (status 10))
 (segment (start 70.062224 59.852208) (end 72.772208 57.142224) (width 0.2032) (layer F.Cu) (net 5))
 (segment (start 72.772208 57.142224) (end 72.772208 56.745746) (width 0.2032) (layer F.Cu) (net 5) (status 20))
 (segment (start 69.735746 64.197792) (end 70.036066 64.498112) (width 0.2032) (layer F.Cu) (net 5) (status 10))
 (segment (start 70.036066 64.498112) (end 70.362544 64.498112) (width 0.2032) (layer F.Cu) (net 5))
 (segment (start 70.362544 64.498112) (end 72.832208 66.967776) (width 0.2032) (layer F.Cu) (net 5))
 (segment (start 72.832208 66.967776) (end 72.832208 67.284254) (width 0.2032) (layer F.Cu) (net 5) (status 20))
 (segment (start 75 65.116462) (end 72.832208 67.284254) (width 0.2032) (layer F.Cu) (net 5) (status 20)))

